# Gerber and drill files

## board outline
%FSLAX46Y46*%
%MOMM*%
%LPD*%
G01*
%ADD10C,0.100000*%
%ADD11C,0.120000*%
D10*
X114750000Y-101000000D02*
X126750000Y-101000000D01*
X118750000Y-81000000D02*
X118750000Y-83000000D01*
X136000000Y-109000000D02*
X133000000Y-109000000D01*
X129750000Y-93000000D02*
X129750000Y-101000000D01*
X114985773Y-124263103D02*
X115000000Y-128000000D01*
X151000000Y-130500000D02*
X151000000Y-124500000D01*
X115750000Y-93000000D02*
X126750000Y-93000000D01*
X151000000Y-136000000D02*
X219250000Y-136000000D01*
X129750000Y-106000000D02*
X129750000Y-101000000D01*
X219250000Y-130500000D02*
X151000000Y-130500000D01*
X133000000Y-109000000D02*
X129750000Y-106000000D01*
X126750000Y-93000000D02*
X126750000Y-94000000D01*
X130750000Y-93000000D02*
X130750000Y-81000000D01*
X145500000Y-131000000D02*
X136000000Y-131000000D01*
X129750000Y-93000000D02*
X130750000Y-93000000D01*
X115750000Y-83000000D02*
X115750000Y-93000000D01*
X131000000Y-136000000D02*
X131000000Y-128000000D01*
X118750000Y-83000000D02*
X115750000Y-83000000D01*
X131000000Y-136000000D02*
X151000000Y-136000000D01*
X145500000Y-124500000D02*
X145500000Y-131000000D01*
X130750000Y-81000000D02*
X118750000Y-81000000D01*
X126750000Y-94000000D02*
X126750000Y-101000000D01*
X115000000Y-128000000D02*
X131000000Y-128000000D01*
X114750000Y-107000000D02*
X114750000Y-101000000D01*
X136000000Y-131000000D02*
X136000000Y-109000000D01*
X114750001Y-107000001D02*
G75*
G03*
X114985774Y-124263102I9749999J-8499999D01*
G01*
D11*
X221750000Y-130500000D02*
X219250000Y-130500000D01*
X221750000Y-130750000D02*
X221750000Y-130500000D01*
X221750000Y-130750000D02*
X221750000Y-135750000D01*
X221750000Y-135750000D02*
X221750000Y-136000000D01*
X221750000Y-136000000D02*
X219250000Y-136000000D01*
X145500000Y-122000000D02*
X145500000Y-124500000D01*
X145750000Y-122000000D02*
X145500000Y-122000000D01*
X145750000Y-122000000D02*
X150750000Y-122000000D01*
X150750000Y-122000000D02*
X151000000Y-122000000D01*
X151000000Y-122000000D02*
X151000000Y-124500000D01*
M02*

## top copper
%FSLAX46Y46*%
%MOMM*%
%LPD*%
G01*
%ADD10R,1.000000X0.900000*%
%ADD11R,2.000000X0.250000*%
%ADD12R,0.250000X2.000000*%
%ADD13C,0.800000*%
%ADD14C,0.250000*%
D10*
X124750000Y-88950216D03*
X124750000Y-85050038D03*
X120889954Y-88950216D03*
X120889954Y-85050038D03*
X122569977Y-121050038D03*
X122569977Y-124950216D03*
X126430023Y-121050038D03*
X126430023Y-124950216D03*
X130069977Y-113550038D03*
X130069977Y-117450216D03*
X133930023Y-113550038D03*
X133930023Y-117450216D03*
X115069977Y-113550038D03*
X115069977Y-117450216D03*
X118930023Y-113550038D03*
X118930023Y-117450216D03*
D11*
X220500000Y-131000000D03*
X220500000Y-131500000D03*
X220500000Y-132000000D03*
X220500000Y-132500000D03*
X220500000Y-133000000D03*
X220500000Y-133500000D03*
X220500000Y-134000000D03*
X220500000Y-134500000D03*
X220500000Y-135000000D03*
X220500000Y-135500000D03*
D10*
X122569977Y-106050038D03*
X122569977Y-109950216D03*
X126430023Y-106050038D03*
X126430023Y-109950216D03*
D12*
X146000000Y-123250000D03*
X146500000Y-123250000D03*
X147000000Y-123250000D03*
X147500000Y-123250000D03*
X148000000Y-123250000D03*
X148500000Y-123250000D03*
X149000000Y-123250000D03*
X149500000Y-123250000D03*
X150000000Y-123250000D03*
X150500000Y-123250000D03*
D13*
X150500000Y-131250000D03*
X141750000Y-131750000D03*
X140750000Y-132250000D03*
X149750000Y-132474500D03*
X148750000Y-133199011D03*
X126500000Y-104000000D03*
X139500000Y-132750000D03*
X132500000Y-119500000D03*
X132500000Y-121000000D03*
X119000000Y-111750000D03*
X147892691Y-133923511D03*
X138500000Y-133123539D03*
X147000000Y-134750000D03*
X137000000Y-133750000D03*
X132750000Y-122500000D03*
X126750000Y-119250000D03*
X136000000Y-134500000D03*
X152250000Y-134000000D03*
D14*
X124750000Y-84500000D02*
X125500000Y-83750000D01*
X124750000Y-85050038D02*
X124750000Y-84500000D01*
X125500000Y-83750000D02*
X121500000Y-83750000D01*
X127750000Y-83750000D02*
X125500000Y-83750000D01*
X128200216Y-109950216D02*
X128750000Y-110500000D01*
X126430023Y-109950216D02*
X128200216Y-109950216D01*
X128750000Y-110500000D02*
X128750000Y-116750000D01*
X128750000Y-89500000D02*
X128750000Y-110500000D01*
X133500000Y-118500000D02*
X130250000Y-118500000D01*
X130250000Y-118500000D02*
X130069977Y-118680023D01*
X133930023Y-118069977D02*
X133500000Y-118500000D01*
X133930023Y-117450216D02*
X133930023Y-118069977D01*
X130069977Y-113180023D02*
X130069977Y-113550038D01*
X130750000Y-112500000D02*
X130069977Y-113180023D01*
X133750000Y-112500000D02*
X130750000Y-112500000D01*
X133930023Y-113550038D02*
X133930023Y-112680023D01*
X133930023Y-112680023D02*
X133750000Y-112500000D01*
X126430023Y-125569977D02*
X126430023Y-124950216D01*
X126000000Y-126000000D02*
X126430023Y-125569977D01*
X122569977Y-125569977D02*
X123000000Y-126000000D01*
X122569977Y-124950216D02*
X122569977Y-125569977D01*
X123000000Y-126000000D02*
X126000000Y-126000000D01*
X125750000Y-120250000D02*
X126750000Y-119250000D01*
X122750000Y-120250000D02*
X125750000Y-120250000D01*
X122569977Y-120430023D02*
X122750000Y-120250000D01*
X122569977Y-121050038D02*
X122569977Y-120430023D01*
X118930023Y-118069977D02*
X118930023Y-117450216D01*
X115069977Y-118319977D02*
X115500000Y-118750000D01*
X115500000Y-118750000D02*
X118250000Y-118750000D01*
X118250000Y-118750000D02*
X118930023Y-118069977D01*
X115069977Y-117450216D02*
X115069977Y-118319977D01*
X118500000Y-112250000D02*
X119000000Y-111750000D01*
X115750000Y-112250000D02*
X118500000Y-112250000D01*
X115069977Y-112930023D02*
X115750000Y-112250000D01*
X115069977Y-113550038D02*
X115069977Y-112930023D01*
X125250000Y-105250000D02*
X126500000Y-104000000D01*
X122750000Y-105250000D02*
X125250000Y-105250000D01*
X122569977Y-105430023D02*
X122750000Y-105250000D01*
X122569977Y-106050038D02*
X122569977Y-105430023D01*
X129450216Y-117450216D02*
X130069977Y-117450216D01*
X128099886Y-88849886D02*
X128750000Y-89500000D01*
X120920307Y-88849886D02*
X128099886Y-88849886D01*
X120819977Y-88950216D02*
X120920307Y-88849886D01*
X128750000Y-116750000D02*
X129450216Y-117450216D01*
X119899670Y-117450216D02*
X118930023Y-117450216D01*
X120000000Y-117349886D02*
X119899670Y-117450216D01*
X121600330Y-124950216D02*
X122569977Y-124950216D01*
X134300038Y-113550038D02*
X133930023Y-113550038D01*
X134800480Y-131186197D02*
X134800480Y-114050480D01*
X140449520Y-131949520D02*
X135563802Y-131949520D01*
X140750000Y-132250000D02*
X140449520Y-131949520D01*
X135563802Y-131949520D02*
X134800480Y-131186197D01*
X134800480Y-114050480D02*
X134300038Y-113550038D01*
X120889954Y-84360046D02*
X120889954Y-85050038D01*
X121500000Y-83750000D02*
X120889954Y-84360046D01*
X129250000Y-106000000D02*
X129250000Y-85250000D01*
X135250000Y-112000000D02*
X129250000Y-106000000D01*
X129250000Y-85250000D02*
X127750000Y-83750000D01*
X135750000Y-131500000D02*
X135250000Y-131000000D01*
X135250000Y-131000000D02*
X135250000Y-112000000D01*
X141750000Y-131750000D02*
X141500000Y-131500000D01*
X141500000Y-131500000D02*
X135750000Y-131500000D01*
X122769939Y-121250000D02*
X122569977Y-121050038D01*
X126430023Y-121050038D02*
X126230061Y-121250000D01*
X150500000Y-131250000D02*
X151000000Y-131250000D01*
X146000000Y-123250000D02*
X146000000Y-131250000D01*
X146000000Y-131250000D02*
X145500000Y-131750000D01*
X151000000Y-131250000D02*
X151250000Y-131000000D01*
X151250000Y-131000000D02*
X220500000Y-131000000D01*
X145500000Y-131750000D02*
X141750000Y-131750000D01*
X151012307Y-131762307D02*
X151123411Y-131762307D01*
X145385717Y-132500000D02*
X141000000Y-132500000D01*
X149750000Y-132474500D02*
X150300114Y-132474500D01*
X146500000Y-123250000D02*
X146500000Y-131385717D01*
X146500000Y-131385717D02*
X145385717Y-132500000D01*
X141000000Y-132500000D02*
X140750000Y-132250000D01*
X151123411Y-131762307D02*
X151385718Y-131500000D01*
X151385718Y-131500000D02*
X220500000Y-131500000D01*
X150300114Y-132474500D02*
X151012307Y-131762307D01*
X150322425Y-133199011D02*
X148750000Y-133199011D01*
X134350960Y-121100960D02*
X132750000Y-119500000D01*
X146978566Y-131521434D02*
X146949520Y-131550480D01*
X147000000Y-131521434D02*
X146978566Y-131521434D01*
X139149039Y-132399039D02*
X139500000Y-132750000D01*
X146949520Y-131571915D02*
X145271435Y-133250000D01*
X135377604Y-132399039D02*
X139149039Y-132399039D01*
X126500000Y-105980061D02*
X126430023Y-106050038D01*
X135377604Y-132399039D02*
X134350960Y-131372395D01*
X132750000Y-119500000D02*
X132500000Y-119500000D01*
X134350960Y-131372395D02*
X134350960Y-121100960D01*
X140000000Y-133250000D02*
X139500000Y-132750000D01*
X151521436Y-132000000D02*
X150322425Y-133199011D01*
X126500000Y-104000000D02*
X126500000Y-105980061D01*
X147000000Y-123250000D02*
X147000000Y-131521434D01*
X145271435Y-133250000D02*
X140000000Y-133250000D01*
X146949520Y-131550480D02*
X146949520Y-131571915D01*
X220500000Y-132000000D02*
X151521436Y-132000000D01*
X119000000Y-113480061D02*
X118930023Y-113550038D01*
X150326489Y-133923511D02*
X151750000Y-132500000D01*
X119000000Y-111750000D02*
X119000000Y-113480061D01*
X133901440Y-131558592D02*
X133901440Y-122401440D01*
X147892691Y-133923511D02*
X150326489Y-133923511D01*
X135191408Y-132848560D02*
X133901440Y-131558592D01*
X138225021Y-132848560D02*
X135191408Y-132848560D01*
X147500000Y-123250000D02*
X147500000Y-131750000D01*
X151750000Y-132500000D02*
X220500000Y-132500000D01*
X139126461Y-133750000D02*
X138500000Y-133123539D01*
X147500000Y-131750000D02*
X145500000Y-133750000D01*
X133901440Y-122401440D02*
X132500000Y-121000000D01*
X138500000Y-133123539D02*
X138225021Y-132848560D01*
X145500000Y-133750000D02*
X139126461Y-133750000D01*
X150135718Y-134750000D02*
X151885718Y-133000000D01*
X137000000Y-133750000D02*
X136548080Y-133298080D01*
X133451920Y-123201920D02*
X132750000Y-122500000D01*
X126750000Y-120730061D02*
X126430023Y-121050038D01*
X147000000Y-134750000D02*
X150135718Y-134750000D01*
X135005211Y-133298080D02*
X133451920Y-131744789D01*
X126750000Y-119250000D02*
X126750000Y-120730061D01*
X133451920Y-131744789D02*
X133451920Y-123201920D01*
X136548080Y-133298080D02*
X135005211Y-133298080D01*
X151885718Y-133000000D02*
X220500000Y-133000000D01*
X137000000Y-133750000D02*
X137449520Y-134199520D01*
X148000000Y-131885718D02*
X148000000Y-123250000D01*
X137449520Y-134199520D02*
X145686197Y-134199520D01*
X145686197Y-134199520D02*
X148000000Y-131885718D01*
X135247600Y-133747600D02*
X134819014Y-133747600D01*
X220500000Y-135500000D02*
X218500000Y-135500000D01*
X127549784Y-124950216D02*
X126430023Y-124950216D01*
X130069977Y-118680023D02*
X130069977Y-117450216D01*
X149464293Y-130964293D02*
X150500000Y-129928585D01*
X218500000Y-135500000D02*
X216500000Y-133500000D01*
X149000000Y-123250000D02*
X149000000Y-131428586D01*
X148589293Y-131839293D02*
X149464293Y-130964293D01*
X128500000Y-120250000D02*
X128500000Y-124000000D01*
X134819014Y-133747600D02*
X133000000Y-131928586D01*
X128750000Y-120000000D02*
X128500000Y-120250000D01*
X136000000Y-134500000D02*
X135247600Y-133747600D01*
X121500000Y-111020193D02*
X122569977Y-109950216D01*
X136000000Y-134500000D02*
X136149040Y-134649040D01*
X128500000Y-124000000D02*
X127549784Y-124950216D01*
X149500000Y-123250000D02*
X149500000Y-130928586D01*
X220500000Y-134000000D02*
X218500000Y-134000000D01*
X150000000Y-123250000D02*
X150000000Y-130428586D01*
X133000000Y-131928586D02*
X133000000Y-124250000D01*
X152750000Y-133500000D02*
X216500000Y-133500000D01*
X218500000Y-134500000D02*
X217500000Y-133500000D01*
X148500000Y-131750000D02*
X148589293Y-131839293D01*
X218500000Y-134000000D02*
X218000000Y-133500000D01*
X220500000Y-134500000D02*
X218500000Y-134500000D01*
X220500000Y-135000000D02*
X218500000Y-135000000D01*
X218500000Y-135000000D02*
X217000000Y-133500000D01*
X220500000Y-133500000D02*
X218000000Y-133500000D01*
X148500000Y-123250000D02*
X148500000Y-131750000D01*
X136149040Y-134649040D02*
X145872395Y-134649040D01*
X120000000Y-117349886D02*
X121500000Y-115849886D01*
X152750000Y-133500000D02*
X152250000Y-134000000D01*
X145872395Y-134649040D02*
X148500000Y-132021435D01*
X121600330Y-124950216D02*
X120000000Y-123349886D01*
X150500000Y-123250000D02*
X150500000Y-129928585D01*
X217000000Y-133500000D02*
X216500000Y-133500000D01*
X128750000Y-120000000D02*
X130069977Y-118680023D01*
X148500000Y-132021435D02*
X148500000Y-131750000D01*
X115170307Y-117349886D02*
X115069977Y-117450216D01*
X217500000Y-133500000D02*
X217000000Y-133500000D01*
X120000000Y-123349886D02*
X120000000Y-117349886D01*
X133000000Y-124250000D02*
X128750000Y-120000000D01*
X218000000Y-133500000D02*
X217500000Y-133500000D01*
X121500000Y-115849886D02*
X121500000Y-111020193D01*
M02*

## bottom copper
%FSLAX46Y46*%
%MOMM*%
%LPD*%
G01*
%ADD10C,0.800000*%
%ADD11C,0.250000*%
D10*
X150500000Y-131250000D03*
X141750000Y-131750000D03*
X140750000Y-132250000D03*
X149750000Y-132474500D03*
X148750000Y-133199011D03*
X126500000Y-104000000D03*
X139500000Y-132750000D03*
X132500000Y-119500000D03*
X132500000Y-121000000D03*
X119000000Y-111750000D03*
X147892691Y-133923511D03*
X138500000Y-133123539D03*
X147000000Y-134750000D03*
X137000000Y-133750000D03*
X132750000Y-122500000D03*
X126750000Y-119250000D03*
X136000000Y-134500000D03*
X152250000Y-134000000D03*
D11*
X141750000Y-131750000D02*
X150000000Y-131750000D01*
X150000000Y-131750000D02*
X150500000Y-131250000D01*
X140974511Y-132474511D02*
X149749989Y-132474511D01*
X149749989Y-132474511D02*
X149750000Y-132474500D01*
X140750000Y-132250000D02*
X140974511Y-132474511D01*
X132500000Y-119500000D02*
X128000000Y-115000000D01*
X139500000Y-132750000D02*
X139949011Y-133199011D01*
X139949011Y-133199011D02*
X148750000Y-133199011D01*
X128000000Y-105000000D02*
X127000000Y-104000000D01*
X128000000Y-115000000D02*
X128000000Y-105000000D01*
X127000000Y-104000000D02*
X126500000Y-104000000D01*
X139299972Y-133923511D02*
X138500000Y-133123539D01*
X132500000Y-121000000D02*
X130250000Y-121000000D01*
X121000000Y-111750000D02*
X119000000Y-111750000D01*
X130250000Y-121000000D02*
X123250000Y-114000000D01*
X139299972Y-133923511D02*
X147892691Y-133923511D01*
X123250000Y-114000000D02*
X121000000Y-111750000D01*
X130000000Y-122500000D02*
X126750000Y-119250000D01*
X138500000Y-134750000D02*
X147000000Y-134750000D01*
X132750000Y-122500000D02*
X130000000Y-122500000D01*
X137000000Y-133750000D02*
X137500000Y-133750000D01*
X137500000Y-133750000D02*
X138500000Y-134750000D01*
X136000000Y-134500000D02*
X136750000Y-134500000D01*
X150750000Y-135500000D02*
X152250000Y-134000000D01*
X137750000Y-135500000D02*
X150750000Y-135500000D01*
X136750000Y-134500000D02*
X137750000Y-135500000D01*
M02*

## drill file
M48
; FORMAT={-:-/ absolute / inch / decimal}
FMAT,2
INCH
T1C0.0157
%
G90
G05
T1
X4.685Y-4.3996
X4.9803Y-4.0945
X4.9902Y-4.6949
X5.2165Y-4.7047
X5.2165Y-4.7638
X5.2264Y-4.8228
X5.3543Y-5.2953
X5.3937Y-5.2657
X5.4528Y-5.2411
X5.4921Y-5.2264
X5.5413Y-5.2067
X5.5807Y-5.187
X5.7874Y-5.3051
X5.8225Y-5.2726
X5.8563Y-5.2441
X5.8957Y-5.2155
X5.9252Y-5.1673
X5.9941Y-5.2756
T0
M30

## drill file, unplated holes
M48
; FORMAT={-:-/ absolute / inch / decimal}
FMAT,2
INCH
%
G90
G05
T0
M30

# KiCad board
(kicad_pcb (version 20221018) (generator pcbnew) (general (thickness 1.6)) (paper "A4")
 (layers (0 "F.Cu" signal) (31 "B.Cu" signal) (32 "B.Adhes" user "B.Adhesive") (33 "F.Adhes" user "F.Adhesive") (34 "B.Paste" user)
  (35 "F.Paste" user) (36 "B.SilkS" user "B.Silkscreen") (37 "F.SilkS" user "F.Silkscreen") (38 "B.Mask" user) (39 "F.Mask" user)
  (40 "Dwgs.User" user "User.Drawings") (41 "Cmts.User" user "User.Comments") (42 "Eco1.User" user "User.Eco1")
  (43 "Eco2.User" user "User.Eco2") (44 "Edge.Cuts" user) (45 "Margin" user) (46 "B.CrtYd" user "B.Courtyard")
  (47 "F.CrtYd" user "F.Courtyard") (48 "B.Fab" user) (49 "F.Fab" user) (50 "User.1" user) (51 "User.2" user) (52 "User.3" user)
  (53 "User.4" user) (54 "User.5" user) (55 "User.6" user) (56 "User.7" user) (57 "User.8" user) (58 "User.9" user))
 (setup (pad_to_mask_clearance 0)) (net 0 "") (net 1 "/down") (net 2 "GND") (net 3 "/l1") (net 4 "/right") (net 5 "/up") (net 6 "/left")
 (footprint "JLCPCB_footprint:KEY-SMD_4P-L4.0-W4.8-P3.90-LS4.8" (layer "F.Cu") (at 124.5 123)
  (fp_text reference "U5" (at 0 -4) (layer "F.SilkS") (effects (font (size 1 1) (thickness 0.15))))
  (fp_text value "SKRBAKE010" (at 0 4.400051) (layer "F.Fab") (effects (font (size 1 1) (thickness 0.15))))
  (pad "1" smd rect (at -1.930023 -1.949962) (size 1 0.9) (layers "F.Cu" "F.Paste" "F.Mask") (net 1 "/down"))
  (pad "2" smd rect (at -1.930023 1.950216) (size 1 0.9) (layers "F.Cu" "F.Paste" "F.Mask") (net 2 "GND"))
  (pad "3" smd rect (at 1.930023 -1.949962) (size 1 0.9) (layers "F.Cu" "F.Paste" "F.Mask") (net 1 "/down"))
  (pad "4" smd rect (at 1.930023 1.950216) (size 1 0.9) (layers "F.Cu" "F.Paste" "F.Mask") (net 2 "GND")))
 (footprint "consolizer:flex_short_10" (layer "F.Cu") (at 220.5 133.5 -90)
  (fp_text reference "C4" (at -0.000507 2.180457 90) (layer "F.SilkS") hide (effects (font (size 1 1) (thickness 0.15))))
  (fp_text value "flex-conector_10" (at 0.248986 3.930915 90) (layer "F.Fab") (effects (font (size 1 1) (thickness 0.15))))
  (fp_line (start -3 -1.25) (end -3 1.25) (stroke (width 0.12) (type solid)) (layer "Edge.Cuts"))
  (fp_line (start -2.75 -1.25) (end -3 -1.25) (stroke (width 0.12) (type solid)) (layer "Edge.Cuts"))
  (fp_line (start -2.75 -1.25) (end 2.25 -1.25) (stroke (width 0.12) (type solid)) (layer "Edge.Cuts"))
  (fp_line (start 2.25 -1.25) (end 2.5 -1.25) (stroke (width 0.12) (type solid)) (layer "Edge.Cuts"))
  (fp_line (start 2.5 -1.25) (end 2.5 1.25) (stroke (width 0.12) (type solid)) (layer "Edge.Cuts"))
  (pad "1" smd rect (at -2.5 0 270) (size 0.25 2) (layers "F.Cu" "F.Paste" "F.Mask") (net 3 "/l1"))
  (pad "2" smd rect (at -2 0 270) (size 0.25 2) (layers "F.Cu" "F.Paste" "F.Mask") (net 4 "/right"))
  (pad "3" smd rect (at -1.5 0 270) (size 0.25 2) (layers "F.Cu" "F.Paste" "F.Mask") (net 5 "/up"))
  (pad "4" smd rect (at -1 0 270) (size 0.25 2) (layers "F.Cu" "F.Paste" "F.Mask") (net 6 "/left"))
  (pad "5" smd rect (at -0.5 0 270) (size 0.25 2) (layers "F.Cu" "F.Paste" "F.Mask") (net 1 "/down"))
  (pad "6" smd rect (at 0 0 270) (size 0.25 2) (layers "F.Cu" "F.Paste" "F.Mask") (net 2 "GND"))
  (pad "7" smd rect (at 0.5 0 270) (size 0.25 2) (layers "F.Cu" "F.Paste" "F.Mask") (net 2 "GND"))
  (pad "8" smd rect (at 1 0 270) (size 0.25 2) (layers "F.Cu" "F.Paste" "F.Mask") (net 2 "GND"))
  (pad "9" smd rect (at 1.5 0 270) (size 0.25 2) (layers "F.Cu" "F.Paste" "F.Mask") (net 2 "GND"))
  (pad "10" smd rect (at 2 0 270) (size 0.25 2) (layers "F.Cu" "F.Paste" "F.Mask") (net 2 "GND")))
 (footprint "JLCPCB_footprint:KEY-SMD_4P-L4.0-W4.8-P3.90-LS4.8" (layer "F.Cu") (at 132 115.5)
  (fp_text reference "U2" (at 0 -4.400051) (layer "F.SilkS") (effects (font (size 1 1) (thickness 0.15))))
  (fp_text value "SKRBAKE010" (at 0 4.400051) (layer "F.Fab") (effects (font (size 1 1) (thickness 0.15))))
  (pad "1" smd rect (at -1.930023 -1.949962) (size 1 0.9) (layers "F.Cu" "F.Paste" "F.Mask") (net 4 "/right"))
  (pad "2" smd rect (at -1.930023 1.950216) (size 1 0.9) (layers "F.Cu" "F.Paste" "F.Mask") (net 2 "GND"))
  (pad "3" smd rect (at 1.930023 -1.949962) (size 1 0.9) (layers "F.Cu" "F.Paste" "F.Mask") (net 4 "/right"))
  (pad "4" smd rect (at 1.930023 1.950216) (size 1 0.9) (layers "F.Cu" "F.Paste" "F.Mask") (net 2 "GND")))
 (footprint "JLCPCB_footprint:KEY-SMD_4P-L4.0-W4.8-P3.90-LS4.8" (layer "F.Cu") (at 122.819977 87)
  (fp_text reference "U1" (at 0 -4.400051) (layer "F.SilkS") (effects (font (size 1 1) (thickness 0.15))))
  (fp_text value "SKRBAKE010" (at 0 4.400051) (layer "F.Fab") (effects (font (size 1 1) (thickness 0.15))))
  (pad "1" smd rect (at -1.930023 -1.949962) (size 1 0.9) (layers "F.Cu" "F.Paste" "F.Mask") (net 3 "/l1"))
  (pad "2" smd rect (at -1.930023 1.950216) (size 1 0.9) (layers "F.Cu" "F.Paste" "F.Mask") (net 2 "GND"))
  (pad "3" smd rect (at 1.930023 -1.949962) (size 1 0.9) (layers "F.Cu" "F.Paste" "F.Mask") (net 3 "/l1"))
  (pad "4" smd rect (at 1.930023 1.950216) (size 1 0.9) (layers "F.Cu" "F.Paste" "F.Mask") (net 2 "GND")))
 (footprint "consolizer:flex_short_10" (layer "F.Cu") (at 148.5 123.25)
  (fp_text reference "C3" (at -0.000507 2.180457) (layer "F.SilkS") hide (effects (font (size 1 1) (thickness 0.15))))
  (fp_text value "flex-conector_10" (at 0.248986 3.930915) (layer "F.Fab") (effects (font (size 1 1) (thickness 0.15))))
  (fp_line (start -3 -1.25) (end -3 1.25) (stroke (width 0.12) (type solid)) (layer "Edge.Cuts"))
  (fp_line (start -2.75 -1.25) (end -3 -1.25) (stroke (width 0.12) (type solid)) (layer "Edge.Cuts"))
  (fp_line (start -2.75 -1.25) (end 2.25 -1.25) (stroke (width 0.12) (type solid)) (layer "Edge.Cuts"))
  (fp_line (start 2.25 -1.25) (end 2.5 -1.25) (stroke (width 0.12) (type solid)) (layer "Edge.Cuts"))
  (fp_line (start 2.5 -1.25) (end 2.5 1.25) (stroke (width 0.12) (type solid)) (layer "Edge.Cuts"))
  (pad "1" smd rect (at -2.5 0) (size 0.25 2) (layers "F.Cu" "F.Paste" "F.Mask") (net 3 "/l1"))
  (pad "2" smd rect (at -2 0) (size 0.25 2) (layers "F.Cu" "F.Paste" "F.Mask") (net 4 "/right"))
  (pad "3" smd rect (at -1.5 0) (size 0.25 2) (layers "F.Cu" "F.Paste" "F.Mask") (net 5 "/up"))
  (pad "4" smd rect (at -1 0) (size 0.25 2) (layers "F.Cu" "F.Paste" "F.Mask") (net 6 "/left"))
  (pad "5" smd rect (at -0.5 0) (size 0.25 2) (layers "F.Cu" "F.Paste" "F.Mask") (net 1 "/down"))
  (pad "6" smd rect (at 0 0) (size 0.25 2) (layers "F.Cu" "F.Paste" "F.Mask") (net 2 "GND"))
  (pad "7" smd rect (at 0.5 0) (size 0.25 2) (layers "F.Cu" "F.Paste" "F.Mask") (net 2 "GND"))
  (pad "8" smd rect (at 1 0) (size 0.25 2) (layers "F.Cu" "F.Paste" "F.Mask") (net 2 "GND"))
  (pad "9" smd rect (at 1.5 0) (size 0.25 2) (layers "F.Cu" "F.Paste" "F.Mask") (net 2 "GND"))
  (pad "10" smd rect (at 2 0) (size 0.25 2) (layers "F.Cu" "F.Paste" "F.Mask") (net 2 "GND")))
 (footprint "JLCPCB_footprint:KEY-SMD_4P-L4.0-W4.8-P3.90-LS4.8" (layer "F.Cu") (at 117 115.5)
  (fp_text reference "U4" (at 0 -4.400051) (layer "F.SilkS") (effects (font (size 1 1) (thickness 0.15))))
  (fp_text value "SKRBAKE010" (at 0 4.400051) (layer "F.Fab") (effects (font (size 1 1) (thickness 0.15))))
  (pad "1" smd rect (at -1.930023 -1.949962) (size 1 0.9) (layers "F.Cu" "F.Paste" "F.Mask") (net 6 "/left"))
  (pad "2" smd rect (at -1.930023 1.950216) (size 1 0.9) (layers "F.Cu" "F.Paste" "F.Mask") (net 2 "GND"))
  (pad "3" smd rect (at 1.930023 -1.949962) (size 1 0.9) (layers "F.Cu" "F.Paste" "F.Mask") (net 6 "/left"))
  (pad "4" smd rect (at 1.930023 1.950216) (size 1 0.9) (layers "F.Cu" "F.Paste" "F.Mask") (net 2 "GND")))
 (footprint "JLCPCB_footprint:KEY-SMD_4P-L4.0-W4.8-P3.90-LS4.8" (layer "F.Cu") (at 124.5 108)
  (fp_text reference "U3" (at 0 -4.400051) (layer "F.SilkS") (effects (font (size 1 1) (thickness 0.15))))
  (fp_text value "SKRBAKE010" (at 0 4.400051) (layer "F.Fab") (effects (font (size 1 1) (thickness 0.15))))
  (pad "1" smd rect (at -1.930023 -1.949962) (size 1 0.9) (layers "F.Cu" "F.Paste" "F.Mask") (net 5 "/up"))
  (pad "2" smd rect (at -1.930023 1.950216) (size 1 0.9) (layers "F.Cu" "F.Paste" "F.Mask") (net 2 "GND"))
  (pad "3" smd rect (at 1.930023 -1.949962) (size 1 0.9) (layers "F.Cu" "F.Paste" "F.Mask") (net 5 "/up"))
  (pad "4" smd rect (at 1.930023 1.950216) (size 1 0.9) (layers "F.Cu" "F.Paste" "F.Mask") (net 2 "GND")))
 (gr_line (start 114.75 101) (end 126.75 101) (stroke (width 0.1) (type solid)) (layer "Edge.Cuts"))
 (gr_line (start 118.75 81) (end 118.75 83) (stroke (width 0.1) (type solid)) (layer "Edge.Cuts"))
 (gr_line (start 136 109) (end 133 109) (stroke (width 0.1) (type solid)) (layer "Edge.Cuts"))
 (gr_line (start 129.75 93) (end 129.75 101) (stroke (width 0.1) (type solid)) (layer "Edge.Cuts"))
 (gr_line (start 114.985773 124.263103) (end 115 128) (stroke (width 0.1) (type solid)) (layer "Edge.Cuts"))
 (gr_line (start 151 130.5) (end 151 124.5) (stroke (width 0.1) (type solid)) (layer "Edge.Cuts"))
 (gr_line (start 115.75 93) (end 126.75 93) (stroke (width 0.1) (type solid)) (layer "Edge.Cuts"))
 (gr_line (start 151 136) (end 219.25 136) (stroke (width 0.1) (type solid)) (layer "Edge.Cuts"))
 (gr_line (start 129.75 106) (end 129.75 101) (stroke (width 0.1) (type solid)) (layer "Edge.Cuts"))
 (gr_line (start 219.25 130.5) (end 151 130.5) (stroke (width 0.1) (type solid)) (layer "Edge.Cuts"))
 (gr_line (start 133 109) (end 129.75 106) (stroke (width 0.1) (type solid)) (layer "Edge.Cuts"))
 (gr_line (start 126.75 93) (end 126.75 94) (stroke (width 0.1) (type solid)) (layer "Edge.Cuts"))
 (gr_line (start 130.75 93) (end 130.75 81) (stroke (width 0.1) (type solid)) (layer "Edge.Cuts"))
 (gr_line (start 145.5 131) (end 136 131) (stroke (width 0.1) (type solid)) (layer "Edge.Cuts"))
 (gr_line (start 129.75 93) (end 130.75 93) (stroke (width 0.1) (type solid)) (layer "Edge.Cuts"))
 (gr_line (start 115.75 83) (end 115.75 93) (stroke (width 0.1) (type solid)) (layer "Edge.Cuts"))
 (gr_line (start 131 136) (end 131 128) (stroke (width 0.1) (type solid)) (layer "Edge.Cuts"))
 (gr_line (start 118.75 83) (end 115.75 83) (stroke (width 0.1) (type solid)) (layer "Edge.Cuts"))
 (gr_line (start 131 136) (end 151 136) (stroke (width 0.1) (type solid)) (layer "Edge.Cuts"))
 (gr_line (start 145.5 124.5) (end 145.5 131) (stroke (width 0.1) (type solid)) (layer "Edge.Cuts"))
 (gr_line (start 130.75 81) (end 118.75 81) (stroke (width 0.1) (type solid)) (layer "Edge.Cuts"))
 (gr_line (start 126.75 94) (end 126.75 101) (stroke (width 0.1) (type solid)) (layer "Edge.Cuts"))
 (gr_line (start 115 128) (end 131 128) (stroke (width 0.1) (type solid)) (layer "Edge.Cuts"))
 (gr_line (start 114.75 107) (end 114.75 101) (stroke (width 0.1) (type solid)) (layer "Edge.Cuts"))
 (gr_line (start 136 131) (end 136 109) (stroke (width 0.1) (type solid)) (layer "Edge.Cuts"))
 (gr_arc (start 114.985773 124.263103) (mid 111.566273 115.676644) (end 114.75 107) (stroke (width 0.1) (type solid)) (layer "Edge.Cuts"))
 (segment (start 121.5 83.75) (end 120.889954 84.360046) (width 0.25) (layer "F.Cu") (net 3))
 (segment (start 150.5 131.25) (end 151 131.25) (width 0.25) (layer "F.Cu") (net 3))
 (segment (start 135.25 113.25) (end 129.25 107.25) (width 0.25) (layer "F.Cu") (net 3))
 (segment (start 125.5 83.75) (end 121.5 83.75) (width 0.25) (layer "F.Cu") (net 3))
 (segment (start 129.25 85.25) (end 127.75 83.75) (width 0.25) (layer "F.Cu") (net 3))
 (segment (start 146 123.25) (end 146 131.25) (width 0.25) (layer "F.Cu") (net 3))
 (segment (start 129.25 107.25) (end 129.25 85.25) (width 0.25) (layer "F.Cu") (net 3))
 (segment (start 146 131.25) (end 145.5 131.75) (width 0.25) (layer "F.Cu") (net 3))
 (segment (start 151 131.25) (end 151.25 131) (width 0.25) (layer "F.Cu") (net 3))
 (segment (start 141.75 131.75) (end 141.5 131.5) (width 0.25) (layer "F.Cu") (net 3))
 (segment (start 124.75 85.050038) (end 124.75 84.5) (width 0.25) (layer "F.Cu") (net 3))
 (segment (start 135.25 131) (end 135.25 113.25) (width 0.25) (layer "F.Cu") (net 3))
 (segment (start 141.5 131.5) (end 135.75 131.5) (width 0.25) (layer "F.Cu") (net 3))
 (segment (start 120.889954 84.360046) (end 120.889954 85.050038) (width 0.25) (layer "F.Cu") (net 3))
 (segment (start 135.75 131.5) (end 135.25 131) (width 0.25) (layer "F.Cu") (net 3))
 (segment (start 124.75 84.5) (end 125.5 83.75) (width 0.25) (layer "F.Cu") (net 3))
 (segment (start 127.75 83.75) (end 125.5 83.75) (width 0.25) (layer "F.Cu") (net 3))
 (segment (start 151.25 131) (end 220.5 131) (width 0.25) (layer "F.Cu") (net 3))
 (segment (start 145.5 131.75) (end 141.75 131.75) (width 0.25) (layer "F.Cu") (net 3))
 (via (at 150.5 131.25) (size 0.8) (drill 0.4) (layers "F.Cu" "B.Cu") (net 3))
 (via (at 141.75 131.75) (size 0.8) (drill 0.4) (layers "F.Cu" "B.Cu") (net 3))
 (segment (start 141.75 131.75) (end 150 131.75) (width 0.25) (layer "B.Cu") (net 3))
 (segment (start 150 131.75) (end 150.5 131.25) (width 0.25) (layer "B.Cu") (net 3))
 (segment (start 151.012307 131.762307) (end 151.123411 131.762307) (width 0.25) (layer "F.Cu") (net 4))
 (segment (start 133.930023 113.550038) (end 133.930023 112.680023) (width 0.25) (layer "F.Cu") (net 4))
 (segment (start 140.44952 131.94952) (end 135.563802 131.94952) (width 0.25) (layer "F.Cu") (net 4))
 (segment (start 134.300038 113.550038) (end 133.930023 113.550038) (width 0.25) (layer "F.Cu") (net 4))
 (segment (start 130.75 112.5) (end 130.069977 113.180023) (width 0.25) (layer "F.Cu") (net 4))
 (segment (start 130.069977 113.180023) (end 130.069977 113.550038) (width 0.25) (layer "F.Cu") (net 4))
 (segment (start 145.385717 132.5) (end 141 132.5) (width 0.25) (layer "F.Cu") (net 4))
 (segment (start 149.75 132.4745) (end 150.300114 132.4745) (width 0.25) (layer "F.Cu") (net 4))
 (segment (start 134.80048 114.05048) (end 134.300038 113.550038) (width 0.25) (layer "F.Cu") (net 4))
 (segment (start 146.5 123.25) (end 146.5 131.385717) (width 0.25) (layer "F.Cu") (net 4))
 (segment (start 135.563802 131.94952) (end 134.80048 131.186197) (width 0.25) (layer "F.Cu") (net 4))
 (segment (start 146.5 131.385717) (end 145.385717 132.5) (width 0.25) (layer "F.Cu") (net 4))
 (segment (start 141 132.5) (end 140.75 132.25) (width 0.25) (layer "F.Cu") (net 4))
 (segment (start 134.80048 131.186197) (end 134.80048 114.05048) (width 0.25) (layer "F.Cu") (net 4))
 (segment (start 151.123411 131.762307) (end 151.385718 131.5) (width 0.25) (layer "F.Cu") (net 4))
 (segment (start 151.385718 131.5) (end 220.5 131.5) (width 0.25) (layer "F.Cu") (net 4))
 (segment (start 140.75 132.25) (end 140.44952 131.94952) (width 0.25) (layer "F.Cu") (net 4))
 (segment (start 133.930023 112.680023) (end 133.75 112.5) (width 0.25) (layer "F.Cu") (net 4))
 (segment (start 133.75 112.5) (end 130.75 112.5) (width 0.25) (layer "F.Cu") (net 4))
 (segment (start 150.300114 132.4745) (end 151.012307 131.762307) (width 0.25) (layer "F.Cu") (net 4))
 (via (at 140.75 132.25) (size 0.8) (drill 0.4) (layers "F.Cu" "B.Cu") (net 4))
 (via (at 149.75 132.4745) (size 0.8) (drill 0.4) (layers "F.Cu" "B.Cu") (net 4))
 (segment (start 140.974511 132.474511) (end 149.749989 132.474511) (width 0.25) (layer "B.Cu") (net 4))
 (segment (start 149.749989 132.474511) (end 149.75 132.4745) (width 0.25) (layer "B.Cu") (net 4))
 (segment (start 140.75 132.25) (end 140.974511 132.474511) (width 0.25) (layer "B.Cu") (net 4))
 (segment (start 150.322425 133.199011) (end 148.75 133.199011) (width 0.25) (layer "F.Cu") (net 5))
 (segment (start 122.569977 106.050038) (end 122.569977 105.430023) (width 0.25) (layer "F.Cu") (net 5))
 (segment (start 134.35096 121.10096) (end 132.75 119.5) (width 0.25) (layer "F.Cu") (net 5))
 (segment (start 146.978566 131.521434) (end 146.94952 131.55048) (width 0.25) (layer "F.Cu") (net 5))
 (segment (start 147 131.521434) (end 146.978566 131.521434) (width 0.25) (layer "F.Cu") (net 5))
 (segment (start 139.149039 132.399039) (end 139.5 132.75) (width 0.25) (layer "F.Cu") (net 5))
 (segment (start 146.94952 131.571915) (end 145.271435 133.25) (width 0.25) (layer "F.Cu") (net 5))
 (segment (start 135.377604 132.399039) (end 139.149039 132.399039) (width 0.25) (layer "F.Cu") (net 5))
 (segment (start 125.25 105.25) (end 126.5 104) (width 0.25) (layer "F.Cu") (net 5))
 (segment (start 122.569977 105.430023) (end 122.75 105.25) (width 0.25) (layer "F.Cu") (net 5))
 (segment (start 126.5 105.980061) (end 126.430023 106.050038) (width 0.25) (layer "F.Cu") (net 5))
 (segment (start 135.377604 132.399039) (end 134.35096 131.372395) (width 0.25) (layer "F.Cu") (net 5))
 (segment (start 132.75 119.5) (end 132.5 119.5) (width 0.25) (layer "F.Cu") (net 5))
 (segment (start 134.35096 131.372395) (end 134.35096 121.10096) (width 0.25) (layer "F.Cu") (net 5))
 (segment (start 140 133.25) (end 139.5 132.75) (width 0.25) (layer "F.Cu") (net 5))
 (segment (start 151.521436 132) (end 150.322425 133.199011) (width 0.25) (layer "F.Cu") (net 5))
 (segment (start 126.5 104) (end 126.5 105.980061) (width 0.25) (layer "F.Cu") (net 5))
 (segment (start 147 123.25) (end 147 131.521434) (width 0.25) (layer "F.Cu") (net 5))
 (segment (start 145.271435 133.25) (end 140 133.25) (width 0.25) (layer "F.Cu") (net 5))
 (segment (start 146.94952 131.55048) (end 146.94952 131.571915) (width 0.25) (layer "F.Cu") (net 5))
 (segment (start 122.75 105.25) (end 125.25 105.25) (width 0.25) (layer "F.Cu") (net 5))
 (segment (start 220.5 132) (end 151.521436 132) (width 0.25) (layer "F.Cu") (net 5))
 (via (at 148.75 133.199011) (size 0.8) (drill 0.4) (layers "F.Cu" "B.Cu") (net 5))
 (via (at 126.5 104) (size 0.8) (drill 0.4) (layers "F.Cu" "B.Cu") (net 5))
 (via (at 139.5 132.75) (size 0.8) (drill 0.4) (layers "F.Cu" "B.Cu") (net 5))
 (via (at 132.5 119.5) (size 0.8) (drill 0.4) (layers "F.Cu" "B.Cu") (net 5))
 (segment (start 132.5 119.5) (end 128 115) (width 0.25) (layer "B.Cu") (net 5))
 (segment (start 139.5 132.75) (end 139.949011 133.199011) (width 0.25) (layer "B.Cu") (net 5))
 (segment (start 139.949011 133.199011) (end 148.75 133.199011) (width 0.25) (layer "B.Cu") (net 5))
 (segment (start 128 105) (end 127 104) (width 0.25) (layer "B.Cu") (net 5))
 (segment (start 128 115) (end 128 105) (width 0.25) (layer "B.Cu") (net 5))
 (segment (start 127 104) (end 126.5 104) (width 0.25) (layer "B.Cu") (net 5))
 (segment (start 119 113.480061) (end 118.930023 113.550038) (width 0.25) (layer "F.Cu") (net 6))
 (segment (start 150.326489 133.923511) (end 151.75 132.5) (width 0.25) (layer "F.Cu") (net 6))
 (segment (start 119 111.75) (end 119 113.480061) (width 0.25) (layer "F.Cu") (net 6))
 (segment (start 118.5 112.25) (end 119 111.75) (width 0.25) (layer "F.Cu") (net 6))
 (segment (start 133.90144 131.558592) (end 133.90144 122.40144) (width 0.25) (layer "F.Cu") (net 6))
 (segment (start 147.892691 133.923511) (end 150.326489 133.923511) (width 0.25) (layer "F.Cu") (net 6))
 (segment (start 115.069977 112.930023) (end 115.75 112.25) (width 0.25) (layer "F.Cu") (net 6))
 (segment (start 135.191408 132.84856) (end 133.90144 131.558592) (width 0.25) (layer "F.Cu") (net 6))
 (segment (start 115.069977 113.550038) (end 115.069977 112.930023) (width 0.25) (layer "F.Cu") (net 6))
 (segment (start 138.225021 132.84856) (end 135.191408 132.84856) (width 0.25) (layer "F.Cu") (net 6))
 (segment (start 147.5 123.25) (end 147.5 131.75) (width 0.25) (layer "F.Cu") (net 6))
 (segment (start 151.75 132.5) (end 220.5 132.5) (width 0.25) (layer "F.Cu") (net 6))
 (segment (start 139.126461 133.75) (end 138.5 133.123539) (width 0.25) (layer "F.Cu") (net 6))
 (segment (start 147.5 131.75) (end 145.5 133.75) (width 0.25) (layer "F.Cu") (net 6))
 (segment (start 115.75 112.25) (end 118.5 112.25) (width 0.25) (layer "F.Cu") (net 6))
 (segment (start 133.90144 122.40144) (end 132.5 121) (width 0.25) (layer "F.Cu") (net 6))
 (segment (start 138.5 133.123539) (end 138.225021 132.84856) (width 0.25) (layer "F.Cu") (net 6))
 (segment (start 145.5 133.75) (end 139.126461 133.75) (width 0.25) (layer "F.Cu") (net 6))
 (via (at 132.5 121) (size 0.8) (drill 0.4) (layers "F.Cu" "B.Cu") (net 6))
 (via (at 119 111.75) (size 0.8) (drill 0.4) (layers "F.Cu" "B.Cu") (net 6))
 (via (at 147.892691 133.923511) (size 0.8) (drill 0.4) (layers "F.Cu" "B.Cu") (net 6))
 (via (at 138.5 133.123539) (size 0.8) (drill 0.4) (layers "F.Cu" "B.Cu") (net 6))
 (segment (start 139.299972 133.923511) (end 138.5 133.123539) (width 0.25) (layer "B.Cu") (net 6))
 (segment (start 132.5 121) (end 130.25 121) (width 0.25) (layer "B.Cu") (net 6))
 (segment (start 121 111.75) (end 119 111.75) (width 0.25) (layer "B.Cu") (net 6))
 (segment (start 130.25 121) (end 123.25 114) (width 0.25) (layer "B.Cu") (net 6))
 (segment (start 139.299972 133.923511) (end 147.892691 133.923511) (width 0.25) (layer "B.Cu") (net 6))
 (segment (start 123.25 114) (end 121 111.75) (width 0.25) (layer "B.Cu") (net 6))
 (segment (start 150.135718 134.75) (end 151.885718 133) (width 0.25) (layer "F.Cu") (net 1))
 (segment (start 126.430023 121.050038) (end 126.230061 121.25) (width 0.25) (layer "F.Cu") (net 1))
 (segment (start 137 133.75) (end 136.54808 133.29808) (width 0.25) (layer "F.Cu") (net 1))
 (segment (start 133.45192 123.20192) (end 132.75 122.5) (width 0.25) (layer "F.Cu") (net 1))
 (segment (start 126.75 120.730061) (end 126.430023 121.050038) (width 0.25) (layer "F.Cu") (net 1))
 (segment (start 147 134.75) (end 150.135718 134.75) (width 0.25) (layer "F.Cu") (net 1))
 (segment (start 122.769939 121.25) (end 122.569977 121.050038) (width 0.25) (layer "F.Cu") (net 1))
 (segment (start 135.005211 133.29808) (end 133.45192 131.744789) (width 0.25) (layer "F.Cu") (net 1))
 (segment (start 125.75 120.25) (end 126.75 119.25) (width 0.25) (layer "F.Cu") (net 1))
 (segment (start 126.75 119.25) (end 126.75 120.730061) (width 0.25) (layer "F.Cu") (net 1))
 (segment (start 133.45192 131.744789) (end 133.45192 123.20192) (width 0.25) (layer "F.Cu") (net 1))
 (segment (start 122.569977 120.430023) (end 122.75 120.25) (width 0.25) (layer "F.Cu") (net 1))
 (segment (start 136.54808 133.29808) (end 135.005211 133.29808) (width 0.25) (layer "F.Cu") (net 1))
 (segment (start 122.569977 121.050038) (end 122.569977 120.430023) (width 0.25) (layer "F.Cu") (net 1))
 (segment (start 151.885718 133) (end 220.5 133) (width 0.25) (layer "F.Cu") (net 1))
 (segment (start 122.75 120.25) (end 125.75 120.25) (width 0.25) (layer "F.Cu") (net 1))
 (segment (start 137 133.75) (end 137.44952 134.19952) (width 0.25) (layer "F.Cu") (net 1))
 (segment (start 148 131.885718) (end 148 123.25) (width 0.25) (layer "F.Cu") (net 1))
 (segment (start 137.44952 134.19952) (end 145.686197 134.19952) (width 0.25) (layer "F.Cu") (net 1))
 (segment (start 145.686197 134.19952) (end 148 131.885718) (width 0.25) (layer "F.Cu") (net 1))
 (via (at 147 134.75) (size 0.8) (drill 0.4) (layers "F.Cu" "B.Cu") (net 1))
 (via (at 137 133.75) (size 0.8) (drill 0.4) (layers "F.Cu" "B.Cu") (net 1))
 (via (at 132.75 122.5) (size 0.8) (drill 0.4) (layers "F.Cu" "B.Cu") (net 1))
 (via (at 126.75 119.25) (size 0.8) (drill 0.4) (layers "F.Cu" "B.Cu") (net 1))
 (segment (start 130 122.5) (end 126.75 119.25) (width 0.25) (layer "B.Cu") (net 1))
 (segment (start 138.5 134.75) (end 147 134.75) (width 0.25) (layer "B.Cu") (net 1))
 (segment (start 132.75 122.5) (end 130 122.5) (width 0.25) (layer "B.Cu") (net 1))
 (segment (start 137 133.75) (end 137.5 133.75) (width 0.25) (layer "B.Cu") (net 1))
 (segment (start 137.5 133.75) (end 138.5 134.75) (width 0.25) (layer "B.Cu") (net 1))
 (segment (start 121.60033 124.950216) (end 122.569977 124.950216) (width 0.25) (layer "F.Cu") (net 2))
 (segment (start 135.2476 133.7476) (end 134.819014 133.7476) (width 0.25) (layer "F.Cu") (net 2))
 (segment (start 220.5 135.5) (end 218.5 135.5) (width 0.25) (layer "F.Cu") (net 2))
 (segment (start 128.099886 88.849886) (end 128.75 89.5) (width 0.25) (layer "F.Cu") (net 2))
 (segment (start 127.549784 124.950216) (end 126.430023 124.950216) (width 0.25) (layer "F.Cu") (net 2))
 (segment (start 130.069977 118.680023) (end 130.069977 117.450216) (width 0.25) (layer "F.Cu") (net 2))
 (segment (start 149.464293 130.964293) (end 150.5 129.928585) (width 0.25) (layer "F.Cu") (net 2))
 (segment (start 218.5 135.5) (end 216.5 133.5) (width 0.25) (layer "F.Cu") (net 2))
 (segment (start 120.819977 88.950216) (end 120.920307 88.849886) (width 0.25) (layer "F.Cu") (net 2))
 (segment (start 128.75 110.5) (end 128.75 116.75) (width 0.25) (layer "F.Cu") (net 2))
 (segment (start 115.069977 117.450216) (end 115.069977 118.319977) (width 0.25) (layer "F.Cu") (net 2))
 (segment (start 149 123.25) (end 149 131.428586) (width 0.25) (layer "F.Cu") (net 2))
 (segment (start 122.569977 124.950216) (end 122.569977 125.569977) (width 0.25) (layer "F.Cu") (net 2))
 (segment (start 120.920307 88.849886) (end 128.099886 88.849886) (width 0.25) (layer "F.Cu") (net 2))
 (segment (start 120 117.349886) (end 119.89967 117.450216) (width 0.25) (layer "F.Cu") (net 2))
 (segment (start 148.589293 131.839293) (end 149.464293 130.964293) (width 0.25) (layer "F.Cu") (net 2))
 (segment (start 122.569977 125.569977) (end 123 126) (width 0.25) (layer "F.Cu") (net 2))
 (segment (start 128.5 120.25) (end 128.5 124) (width 0.25) (layer "F.Cu") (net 2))
 (segment (start 134.819014 133.7476) (end 133 131.928586) (width 0.25) (layer "F.Cu") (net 2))
 (segment (start 128.75 120) (end 128.5 120.25) (width 0.25) (layer "F.Cu") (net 2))
 (segment (start 136 134.5) (end 135.2476 133.7476) (width 0.25) (layer "F.Cu") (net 2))
 (segment (start 129.450216 117.450216) (end 130.069977 117.450216) (width 0.25) (layer "F.Cu") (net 2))
 (segment (start 118.25 118.75) (end 118.930023 118.069977) (width 0.25) (layer "F.Cu") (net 2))
 (segment (start 121.5 111.020193) (end 122.569977 109.950216) (width 0.25) (layer "F.Cu") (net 2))
 (segment (start 128.75 89.5) (end 128.75 110.5) (width 0.25) (layer "F.Cu") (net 2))
 (segment (start 136 134.5) (end 136.14904 134.64904) (width 0.25) (layer "F.Cu") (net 2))
 (segment (start 128.5 124) (end 127.549784 124.950216) (width 0.25) (layer "F.Cu") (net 2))
 (segment (start 119.89967 117.450216) (end 118.930023 117.450216) (width 0.25) (layer "F.Cu") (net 2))
 (segment (start 115.069977 118.319977) (end 115.5 118.75) (width 0.25) (layer "F.Cu") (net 2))
 (segment (start 149.5 123.25) (end 149.5 130.928586) (width 0.25) (layer "F.Cu") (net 2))
 (segment (start 220.5 134) (end 218.5 134) (width 0.25) (layer "F.Cu") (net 2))
 (segment (start 150 123.25) (end 150 130.428586) (width 0.25) (layer "F.Cu") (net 2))
 (segment (start 128.75 116.75) (end 129.450216 117.450216) (width 0.25) (layer "F.Cu") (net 2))
 (segment (start 133 131.928586) (end 133 124.25) (width 0.25) (layer "F.Cu") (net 2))
 (segment (start 128.200216 109.950216) (end 128.75 110.5) (width 0.25) (layer "F.Cu") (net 2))
 (segment (start 152.75 133.5) (end 216.5 133.5) (width 0.25) (layer "F.Cu") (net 2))
 (segment (start 133.930023 117.450216) (end 133.930023 118.069977) (width 0.25) (layer "F.Cu") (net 2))
 (segment (start 218.5 134.5) (end 217.5 133.5) (width 0.25) (layer "F.Cu") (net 2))
 (segment (start 148.5 131.75) (end 148.589293 131.839293) (width 0.25) (layer "F.Cu") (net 2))
 (segment (start 218.5 134) (end 218 133.5) (width 0.25) (layer "F.Cu") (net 2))
 (segment (start 220.5 134.5) (end 218.5 134.5) (width 0.25) (layer "F.Cu") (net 2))
 (segment (start 220.5 135) (end 218.5 135) (width 0.25) (layer "F.Cu") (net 2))
 (segment (start 218.5 135) (end 217 133.5) (width 0.25) (layer "F.Cu") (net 2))
 (segment (start 220.5 133.5) (end 218 133.5) (width 0.25) (layer "F.Cu") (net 2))
 (segment (start 148.5 123.25) (end 148.5 131.75) (width 0.25) (layer "F.Cu") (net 2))
 (segment (start 136.14904 134.64904) (end 145.872395 134.64904) (width 0.25) (layer "F.Cu") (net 2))
 (segment (start 115.5 118.75) (end 118.25 118.75) (width 0.25) (layer "F.Cu") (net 2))
 (segment (start 130.25 118.5) (end 130.069977 118.680023) (width 0.25) (layer "F.Cu") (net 2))
 (segment (start 120 117.349886) (end 121.5 115.849886) (width 0.25) (layer "F.Cu") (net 2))
 (segment (start 152.75 133.5) (end 152.25 134) (width 0.25) (layer "F.Cu") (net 2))
 (segment (start 145.872395 134.64904) (end 148.5 132.021435) (width 0.25) (layer "F.Cu") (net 2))
 (segment (start 126.430023 109.950216) (end 128.200216 109.950216) (width 0.25) (layer "F.Cu") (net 2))
 (segment (start 121.60033 124.950216) (end 120 123.349886) (width 0.25) (layer "F.Cu") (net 2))
 (segment (start 126.430023 125.569977) (end 126.430023 124.950216) (width 0.25) (layer "F.Cu") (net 2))
 (segment (start 150.5 123.25) (end 150.5 129.928585) (width 0.25) (layer "F.Cu") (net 2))
 (segment (start 217 133.5) (end 216.5 133.5) (width 0.25) (layer "F.Cu") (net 2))
 (segment (start 128.75 120) (end 130.069977 118.680023) (width 0.25) (layer "F.Cu") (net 2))
 (segment (start 148.5 132.021435) (end 148.5 131.75) (width 0.25) (layer "F.Cu") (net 2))
 (segment (start 115.170307 117.349886) (end 115.069977 117.450216) (width 0.25) (layer "F.Cu") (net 2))
 (segment (start 217.5 133.5) (end 217 133.5) (width 0.25) (layer "F.Cu") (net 2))
 (segment (start 118.930023 118.069977) (end 118.930023 117.450216) (width 0.25) (layer "F.Cu") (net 2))
 (segment (start 126 126) (end 126.430023 125.569977) (width 0.25) (layer "F.Cu") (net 2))
 (segment (start 120 123.349886) (end 120 117.349886) (width 0.25) (layer "F.Cu") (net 2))
 (segment (start 133 124.25) (end 128.75 120) (width 0.25) (layer "F.Cu") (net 2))
 (segment (start 133.5 118.5) (end 130.25 118.5) (width 0.25) (layer "F.Cu") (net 2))
 (segment (start 218 133.5) (end 217.5 133.5) (width 0.25) (layer "F.Cu") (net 2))
 (segment (start 121.5 115.849886) (end 121.5 111.020193) (width 0.25) (layer "F.Cu") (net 2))
 (segment (start 123 126) (end 126 126) (width 0.25) (layer "F.Cu") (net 2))
 (segment (start 133.930023 118.069977) (end 133.5 118.5) (width 0.25) (layer "F.Cu") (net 2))
 (via (at 136 134.5) (size 0.8) (drill 0.4) (layers "F.Cu" "B.Cu") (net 2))
 (via (at 152.25 134) (size 0.8) (drill 0.4) (layers "F.Cu" "B.Cu") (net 2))
 (segment (start 136 134.5) (end 136.75 134.5) (width 0.25) (layer "B.Cu") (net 2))
 (segment (start 150.75 135.5) (end 152.25 134) (width 0.25) (layer "B.Cu") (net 2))
 (segment (start 137.75 135.5) (end 150.75 135.5) (width 0.25) (layer "B.Cu") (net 2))
 (segment (start 136.75 134.5) (end 137.75 135.5) (width 0.25) (layer "B.Cu") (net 2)))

